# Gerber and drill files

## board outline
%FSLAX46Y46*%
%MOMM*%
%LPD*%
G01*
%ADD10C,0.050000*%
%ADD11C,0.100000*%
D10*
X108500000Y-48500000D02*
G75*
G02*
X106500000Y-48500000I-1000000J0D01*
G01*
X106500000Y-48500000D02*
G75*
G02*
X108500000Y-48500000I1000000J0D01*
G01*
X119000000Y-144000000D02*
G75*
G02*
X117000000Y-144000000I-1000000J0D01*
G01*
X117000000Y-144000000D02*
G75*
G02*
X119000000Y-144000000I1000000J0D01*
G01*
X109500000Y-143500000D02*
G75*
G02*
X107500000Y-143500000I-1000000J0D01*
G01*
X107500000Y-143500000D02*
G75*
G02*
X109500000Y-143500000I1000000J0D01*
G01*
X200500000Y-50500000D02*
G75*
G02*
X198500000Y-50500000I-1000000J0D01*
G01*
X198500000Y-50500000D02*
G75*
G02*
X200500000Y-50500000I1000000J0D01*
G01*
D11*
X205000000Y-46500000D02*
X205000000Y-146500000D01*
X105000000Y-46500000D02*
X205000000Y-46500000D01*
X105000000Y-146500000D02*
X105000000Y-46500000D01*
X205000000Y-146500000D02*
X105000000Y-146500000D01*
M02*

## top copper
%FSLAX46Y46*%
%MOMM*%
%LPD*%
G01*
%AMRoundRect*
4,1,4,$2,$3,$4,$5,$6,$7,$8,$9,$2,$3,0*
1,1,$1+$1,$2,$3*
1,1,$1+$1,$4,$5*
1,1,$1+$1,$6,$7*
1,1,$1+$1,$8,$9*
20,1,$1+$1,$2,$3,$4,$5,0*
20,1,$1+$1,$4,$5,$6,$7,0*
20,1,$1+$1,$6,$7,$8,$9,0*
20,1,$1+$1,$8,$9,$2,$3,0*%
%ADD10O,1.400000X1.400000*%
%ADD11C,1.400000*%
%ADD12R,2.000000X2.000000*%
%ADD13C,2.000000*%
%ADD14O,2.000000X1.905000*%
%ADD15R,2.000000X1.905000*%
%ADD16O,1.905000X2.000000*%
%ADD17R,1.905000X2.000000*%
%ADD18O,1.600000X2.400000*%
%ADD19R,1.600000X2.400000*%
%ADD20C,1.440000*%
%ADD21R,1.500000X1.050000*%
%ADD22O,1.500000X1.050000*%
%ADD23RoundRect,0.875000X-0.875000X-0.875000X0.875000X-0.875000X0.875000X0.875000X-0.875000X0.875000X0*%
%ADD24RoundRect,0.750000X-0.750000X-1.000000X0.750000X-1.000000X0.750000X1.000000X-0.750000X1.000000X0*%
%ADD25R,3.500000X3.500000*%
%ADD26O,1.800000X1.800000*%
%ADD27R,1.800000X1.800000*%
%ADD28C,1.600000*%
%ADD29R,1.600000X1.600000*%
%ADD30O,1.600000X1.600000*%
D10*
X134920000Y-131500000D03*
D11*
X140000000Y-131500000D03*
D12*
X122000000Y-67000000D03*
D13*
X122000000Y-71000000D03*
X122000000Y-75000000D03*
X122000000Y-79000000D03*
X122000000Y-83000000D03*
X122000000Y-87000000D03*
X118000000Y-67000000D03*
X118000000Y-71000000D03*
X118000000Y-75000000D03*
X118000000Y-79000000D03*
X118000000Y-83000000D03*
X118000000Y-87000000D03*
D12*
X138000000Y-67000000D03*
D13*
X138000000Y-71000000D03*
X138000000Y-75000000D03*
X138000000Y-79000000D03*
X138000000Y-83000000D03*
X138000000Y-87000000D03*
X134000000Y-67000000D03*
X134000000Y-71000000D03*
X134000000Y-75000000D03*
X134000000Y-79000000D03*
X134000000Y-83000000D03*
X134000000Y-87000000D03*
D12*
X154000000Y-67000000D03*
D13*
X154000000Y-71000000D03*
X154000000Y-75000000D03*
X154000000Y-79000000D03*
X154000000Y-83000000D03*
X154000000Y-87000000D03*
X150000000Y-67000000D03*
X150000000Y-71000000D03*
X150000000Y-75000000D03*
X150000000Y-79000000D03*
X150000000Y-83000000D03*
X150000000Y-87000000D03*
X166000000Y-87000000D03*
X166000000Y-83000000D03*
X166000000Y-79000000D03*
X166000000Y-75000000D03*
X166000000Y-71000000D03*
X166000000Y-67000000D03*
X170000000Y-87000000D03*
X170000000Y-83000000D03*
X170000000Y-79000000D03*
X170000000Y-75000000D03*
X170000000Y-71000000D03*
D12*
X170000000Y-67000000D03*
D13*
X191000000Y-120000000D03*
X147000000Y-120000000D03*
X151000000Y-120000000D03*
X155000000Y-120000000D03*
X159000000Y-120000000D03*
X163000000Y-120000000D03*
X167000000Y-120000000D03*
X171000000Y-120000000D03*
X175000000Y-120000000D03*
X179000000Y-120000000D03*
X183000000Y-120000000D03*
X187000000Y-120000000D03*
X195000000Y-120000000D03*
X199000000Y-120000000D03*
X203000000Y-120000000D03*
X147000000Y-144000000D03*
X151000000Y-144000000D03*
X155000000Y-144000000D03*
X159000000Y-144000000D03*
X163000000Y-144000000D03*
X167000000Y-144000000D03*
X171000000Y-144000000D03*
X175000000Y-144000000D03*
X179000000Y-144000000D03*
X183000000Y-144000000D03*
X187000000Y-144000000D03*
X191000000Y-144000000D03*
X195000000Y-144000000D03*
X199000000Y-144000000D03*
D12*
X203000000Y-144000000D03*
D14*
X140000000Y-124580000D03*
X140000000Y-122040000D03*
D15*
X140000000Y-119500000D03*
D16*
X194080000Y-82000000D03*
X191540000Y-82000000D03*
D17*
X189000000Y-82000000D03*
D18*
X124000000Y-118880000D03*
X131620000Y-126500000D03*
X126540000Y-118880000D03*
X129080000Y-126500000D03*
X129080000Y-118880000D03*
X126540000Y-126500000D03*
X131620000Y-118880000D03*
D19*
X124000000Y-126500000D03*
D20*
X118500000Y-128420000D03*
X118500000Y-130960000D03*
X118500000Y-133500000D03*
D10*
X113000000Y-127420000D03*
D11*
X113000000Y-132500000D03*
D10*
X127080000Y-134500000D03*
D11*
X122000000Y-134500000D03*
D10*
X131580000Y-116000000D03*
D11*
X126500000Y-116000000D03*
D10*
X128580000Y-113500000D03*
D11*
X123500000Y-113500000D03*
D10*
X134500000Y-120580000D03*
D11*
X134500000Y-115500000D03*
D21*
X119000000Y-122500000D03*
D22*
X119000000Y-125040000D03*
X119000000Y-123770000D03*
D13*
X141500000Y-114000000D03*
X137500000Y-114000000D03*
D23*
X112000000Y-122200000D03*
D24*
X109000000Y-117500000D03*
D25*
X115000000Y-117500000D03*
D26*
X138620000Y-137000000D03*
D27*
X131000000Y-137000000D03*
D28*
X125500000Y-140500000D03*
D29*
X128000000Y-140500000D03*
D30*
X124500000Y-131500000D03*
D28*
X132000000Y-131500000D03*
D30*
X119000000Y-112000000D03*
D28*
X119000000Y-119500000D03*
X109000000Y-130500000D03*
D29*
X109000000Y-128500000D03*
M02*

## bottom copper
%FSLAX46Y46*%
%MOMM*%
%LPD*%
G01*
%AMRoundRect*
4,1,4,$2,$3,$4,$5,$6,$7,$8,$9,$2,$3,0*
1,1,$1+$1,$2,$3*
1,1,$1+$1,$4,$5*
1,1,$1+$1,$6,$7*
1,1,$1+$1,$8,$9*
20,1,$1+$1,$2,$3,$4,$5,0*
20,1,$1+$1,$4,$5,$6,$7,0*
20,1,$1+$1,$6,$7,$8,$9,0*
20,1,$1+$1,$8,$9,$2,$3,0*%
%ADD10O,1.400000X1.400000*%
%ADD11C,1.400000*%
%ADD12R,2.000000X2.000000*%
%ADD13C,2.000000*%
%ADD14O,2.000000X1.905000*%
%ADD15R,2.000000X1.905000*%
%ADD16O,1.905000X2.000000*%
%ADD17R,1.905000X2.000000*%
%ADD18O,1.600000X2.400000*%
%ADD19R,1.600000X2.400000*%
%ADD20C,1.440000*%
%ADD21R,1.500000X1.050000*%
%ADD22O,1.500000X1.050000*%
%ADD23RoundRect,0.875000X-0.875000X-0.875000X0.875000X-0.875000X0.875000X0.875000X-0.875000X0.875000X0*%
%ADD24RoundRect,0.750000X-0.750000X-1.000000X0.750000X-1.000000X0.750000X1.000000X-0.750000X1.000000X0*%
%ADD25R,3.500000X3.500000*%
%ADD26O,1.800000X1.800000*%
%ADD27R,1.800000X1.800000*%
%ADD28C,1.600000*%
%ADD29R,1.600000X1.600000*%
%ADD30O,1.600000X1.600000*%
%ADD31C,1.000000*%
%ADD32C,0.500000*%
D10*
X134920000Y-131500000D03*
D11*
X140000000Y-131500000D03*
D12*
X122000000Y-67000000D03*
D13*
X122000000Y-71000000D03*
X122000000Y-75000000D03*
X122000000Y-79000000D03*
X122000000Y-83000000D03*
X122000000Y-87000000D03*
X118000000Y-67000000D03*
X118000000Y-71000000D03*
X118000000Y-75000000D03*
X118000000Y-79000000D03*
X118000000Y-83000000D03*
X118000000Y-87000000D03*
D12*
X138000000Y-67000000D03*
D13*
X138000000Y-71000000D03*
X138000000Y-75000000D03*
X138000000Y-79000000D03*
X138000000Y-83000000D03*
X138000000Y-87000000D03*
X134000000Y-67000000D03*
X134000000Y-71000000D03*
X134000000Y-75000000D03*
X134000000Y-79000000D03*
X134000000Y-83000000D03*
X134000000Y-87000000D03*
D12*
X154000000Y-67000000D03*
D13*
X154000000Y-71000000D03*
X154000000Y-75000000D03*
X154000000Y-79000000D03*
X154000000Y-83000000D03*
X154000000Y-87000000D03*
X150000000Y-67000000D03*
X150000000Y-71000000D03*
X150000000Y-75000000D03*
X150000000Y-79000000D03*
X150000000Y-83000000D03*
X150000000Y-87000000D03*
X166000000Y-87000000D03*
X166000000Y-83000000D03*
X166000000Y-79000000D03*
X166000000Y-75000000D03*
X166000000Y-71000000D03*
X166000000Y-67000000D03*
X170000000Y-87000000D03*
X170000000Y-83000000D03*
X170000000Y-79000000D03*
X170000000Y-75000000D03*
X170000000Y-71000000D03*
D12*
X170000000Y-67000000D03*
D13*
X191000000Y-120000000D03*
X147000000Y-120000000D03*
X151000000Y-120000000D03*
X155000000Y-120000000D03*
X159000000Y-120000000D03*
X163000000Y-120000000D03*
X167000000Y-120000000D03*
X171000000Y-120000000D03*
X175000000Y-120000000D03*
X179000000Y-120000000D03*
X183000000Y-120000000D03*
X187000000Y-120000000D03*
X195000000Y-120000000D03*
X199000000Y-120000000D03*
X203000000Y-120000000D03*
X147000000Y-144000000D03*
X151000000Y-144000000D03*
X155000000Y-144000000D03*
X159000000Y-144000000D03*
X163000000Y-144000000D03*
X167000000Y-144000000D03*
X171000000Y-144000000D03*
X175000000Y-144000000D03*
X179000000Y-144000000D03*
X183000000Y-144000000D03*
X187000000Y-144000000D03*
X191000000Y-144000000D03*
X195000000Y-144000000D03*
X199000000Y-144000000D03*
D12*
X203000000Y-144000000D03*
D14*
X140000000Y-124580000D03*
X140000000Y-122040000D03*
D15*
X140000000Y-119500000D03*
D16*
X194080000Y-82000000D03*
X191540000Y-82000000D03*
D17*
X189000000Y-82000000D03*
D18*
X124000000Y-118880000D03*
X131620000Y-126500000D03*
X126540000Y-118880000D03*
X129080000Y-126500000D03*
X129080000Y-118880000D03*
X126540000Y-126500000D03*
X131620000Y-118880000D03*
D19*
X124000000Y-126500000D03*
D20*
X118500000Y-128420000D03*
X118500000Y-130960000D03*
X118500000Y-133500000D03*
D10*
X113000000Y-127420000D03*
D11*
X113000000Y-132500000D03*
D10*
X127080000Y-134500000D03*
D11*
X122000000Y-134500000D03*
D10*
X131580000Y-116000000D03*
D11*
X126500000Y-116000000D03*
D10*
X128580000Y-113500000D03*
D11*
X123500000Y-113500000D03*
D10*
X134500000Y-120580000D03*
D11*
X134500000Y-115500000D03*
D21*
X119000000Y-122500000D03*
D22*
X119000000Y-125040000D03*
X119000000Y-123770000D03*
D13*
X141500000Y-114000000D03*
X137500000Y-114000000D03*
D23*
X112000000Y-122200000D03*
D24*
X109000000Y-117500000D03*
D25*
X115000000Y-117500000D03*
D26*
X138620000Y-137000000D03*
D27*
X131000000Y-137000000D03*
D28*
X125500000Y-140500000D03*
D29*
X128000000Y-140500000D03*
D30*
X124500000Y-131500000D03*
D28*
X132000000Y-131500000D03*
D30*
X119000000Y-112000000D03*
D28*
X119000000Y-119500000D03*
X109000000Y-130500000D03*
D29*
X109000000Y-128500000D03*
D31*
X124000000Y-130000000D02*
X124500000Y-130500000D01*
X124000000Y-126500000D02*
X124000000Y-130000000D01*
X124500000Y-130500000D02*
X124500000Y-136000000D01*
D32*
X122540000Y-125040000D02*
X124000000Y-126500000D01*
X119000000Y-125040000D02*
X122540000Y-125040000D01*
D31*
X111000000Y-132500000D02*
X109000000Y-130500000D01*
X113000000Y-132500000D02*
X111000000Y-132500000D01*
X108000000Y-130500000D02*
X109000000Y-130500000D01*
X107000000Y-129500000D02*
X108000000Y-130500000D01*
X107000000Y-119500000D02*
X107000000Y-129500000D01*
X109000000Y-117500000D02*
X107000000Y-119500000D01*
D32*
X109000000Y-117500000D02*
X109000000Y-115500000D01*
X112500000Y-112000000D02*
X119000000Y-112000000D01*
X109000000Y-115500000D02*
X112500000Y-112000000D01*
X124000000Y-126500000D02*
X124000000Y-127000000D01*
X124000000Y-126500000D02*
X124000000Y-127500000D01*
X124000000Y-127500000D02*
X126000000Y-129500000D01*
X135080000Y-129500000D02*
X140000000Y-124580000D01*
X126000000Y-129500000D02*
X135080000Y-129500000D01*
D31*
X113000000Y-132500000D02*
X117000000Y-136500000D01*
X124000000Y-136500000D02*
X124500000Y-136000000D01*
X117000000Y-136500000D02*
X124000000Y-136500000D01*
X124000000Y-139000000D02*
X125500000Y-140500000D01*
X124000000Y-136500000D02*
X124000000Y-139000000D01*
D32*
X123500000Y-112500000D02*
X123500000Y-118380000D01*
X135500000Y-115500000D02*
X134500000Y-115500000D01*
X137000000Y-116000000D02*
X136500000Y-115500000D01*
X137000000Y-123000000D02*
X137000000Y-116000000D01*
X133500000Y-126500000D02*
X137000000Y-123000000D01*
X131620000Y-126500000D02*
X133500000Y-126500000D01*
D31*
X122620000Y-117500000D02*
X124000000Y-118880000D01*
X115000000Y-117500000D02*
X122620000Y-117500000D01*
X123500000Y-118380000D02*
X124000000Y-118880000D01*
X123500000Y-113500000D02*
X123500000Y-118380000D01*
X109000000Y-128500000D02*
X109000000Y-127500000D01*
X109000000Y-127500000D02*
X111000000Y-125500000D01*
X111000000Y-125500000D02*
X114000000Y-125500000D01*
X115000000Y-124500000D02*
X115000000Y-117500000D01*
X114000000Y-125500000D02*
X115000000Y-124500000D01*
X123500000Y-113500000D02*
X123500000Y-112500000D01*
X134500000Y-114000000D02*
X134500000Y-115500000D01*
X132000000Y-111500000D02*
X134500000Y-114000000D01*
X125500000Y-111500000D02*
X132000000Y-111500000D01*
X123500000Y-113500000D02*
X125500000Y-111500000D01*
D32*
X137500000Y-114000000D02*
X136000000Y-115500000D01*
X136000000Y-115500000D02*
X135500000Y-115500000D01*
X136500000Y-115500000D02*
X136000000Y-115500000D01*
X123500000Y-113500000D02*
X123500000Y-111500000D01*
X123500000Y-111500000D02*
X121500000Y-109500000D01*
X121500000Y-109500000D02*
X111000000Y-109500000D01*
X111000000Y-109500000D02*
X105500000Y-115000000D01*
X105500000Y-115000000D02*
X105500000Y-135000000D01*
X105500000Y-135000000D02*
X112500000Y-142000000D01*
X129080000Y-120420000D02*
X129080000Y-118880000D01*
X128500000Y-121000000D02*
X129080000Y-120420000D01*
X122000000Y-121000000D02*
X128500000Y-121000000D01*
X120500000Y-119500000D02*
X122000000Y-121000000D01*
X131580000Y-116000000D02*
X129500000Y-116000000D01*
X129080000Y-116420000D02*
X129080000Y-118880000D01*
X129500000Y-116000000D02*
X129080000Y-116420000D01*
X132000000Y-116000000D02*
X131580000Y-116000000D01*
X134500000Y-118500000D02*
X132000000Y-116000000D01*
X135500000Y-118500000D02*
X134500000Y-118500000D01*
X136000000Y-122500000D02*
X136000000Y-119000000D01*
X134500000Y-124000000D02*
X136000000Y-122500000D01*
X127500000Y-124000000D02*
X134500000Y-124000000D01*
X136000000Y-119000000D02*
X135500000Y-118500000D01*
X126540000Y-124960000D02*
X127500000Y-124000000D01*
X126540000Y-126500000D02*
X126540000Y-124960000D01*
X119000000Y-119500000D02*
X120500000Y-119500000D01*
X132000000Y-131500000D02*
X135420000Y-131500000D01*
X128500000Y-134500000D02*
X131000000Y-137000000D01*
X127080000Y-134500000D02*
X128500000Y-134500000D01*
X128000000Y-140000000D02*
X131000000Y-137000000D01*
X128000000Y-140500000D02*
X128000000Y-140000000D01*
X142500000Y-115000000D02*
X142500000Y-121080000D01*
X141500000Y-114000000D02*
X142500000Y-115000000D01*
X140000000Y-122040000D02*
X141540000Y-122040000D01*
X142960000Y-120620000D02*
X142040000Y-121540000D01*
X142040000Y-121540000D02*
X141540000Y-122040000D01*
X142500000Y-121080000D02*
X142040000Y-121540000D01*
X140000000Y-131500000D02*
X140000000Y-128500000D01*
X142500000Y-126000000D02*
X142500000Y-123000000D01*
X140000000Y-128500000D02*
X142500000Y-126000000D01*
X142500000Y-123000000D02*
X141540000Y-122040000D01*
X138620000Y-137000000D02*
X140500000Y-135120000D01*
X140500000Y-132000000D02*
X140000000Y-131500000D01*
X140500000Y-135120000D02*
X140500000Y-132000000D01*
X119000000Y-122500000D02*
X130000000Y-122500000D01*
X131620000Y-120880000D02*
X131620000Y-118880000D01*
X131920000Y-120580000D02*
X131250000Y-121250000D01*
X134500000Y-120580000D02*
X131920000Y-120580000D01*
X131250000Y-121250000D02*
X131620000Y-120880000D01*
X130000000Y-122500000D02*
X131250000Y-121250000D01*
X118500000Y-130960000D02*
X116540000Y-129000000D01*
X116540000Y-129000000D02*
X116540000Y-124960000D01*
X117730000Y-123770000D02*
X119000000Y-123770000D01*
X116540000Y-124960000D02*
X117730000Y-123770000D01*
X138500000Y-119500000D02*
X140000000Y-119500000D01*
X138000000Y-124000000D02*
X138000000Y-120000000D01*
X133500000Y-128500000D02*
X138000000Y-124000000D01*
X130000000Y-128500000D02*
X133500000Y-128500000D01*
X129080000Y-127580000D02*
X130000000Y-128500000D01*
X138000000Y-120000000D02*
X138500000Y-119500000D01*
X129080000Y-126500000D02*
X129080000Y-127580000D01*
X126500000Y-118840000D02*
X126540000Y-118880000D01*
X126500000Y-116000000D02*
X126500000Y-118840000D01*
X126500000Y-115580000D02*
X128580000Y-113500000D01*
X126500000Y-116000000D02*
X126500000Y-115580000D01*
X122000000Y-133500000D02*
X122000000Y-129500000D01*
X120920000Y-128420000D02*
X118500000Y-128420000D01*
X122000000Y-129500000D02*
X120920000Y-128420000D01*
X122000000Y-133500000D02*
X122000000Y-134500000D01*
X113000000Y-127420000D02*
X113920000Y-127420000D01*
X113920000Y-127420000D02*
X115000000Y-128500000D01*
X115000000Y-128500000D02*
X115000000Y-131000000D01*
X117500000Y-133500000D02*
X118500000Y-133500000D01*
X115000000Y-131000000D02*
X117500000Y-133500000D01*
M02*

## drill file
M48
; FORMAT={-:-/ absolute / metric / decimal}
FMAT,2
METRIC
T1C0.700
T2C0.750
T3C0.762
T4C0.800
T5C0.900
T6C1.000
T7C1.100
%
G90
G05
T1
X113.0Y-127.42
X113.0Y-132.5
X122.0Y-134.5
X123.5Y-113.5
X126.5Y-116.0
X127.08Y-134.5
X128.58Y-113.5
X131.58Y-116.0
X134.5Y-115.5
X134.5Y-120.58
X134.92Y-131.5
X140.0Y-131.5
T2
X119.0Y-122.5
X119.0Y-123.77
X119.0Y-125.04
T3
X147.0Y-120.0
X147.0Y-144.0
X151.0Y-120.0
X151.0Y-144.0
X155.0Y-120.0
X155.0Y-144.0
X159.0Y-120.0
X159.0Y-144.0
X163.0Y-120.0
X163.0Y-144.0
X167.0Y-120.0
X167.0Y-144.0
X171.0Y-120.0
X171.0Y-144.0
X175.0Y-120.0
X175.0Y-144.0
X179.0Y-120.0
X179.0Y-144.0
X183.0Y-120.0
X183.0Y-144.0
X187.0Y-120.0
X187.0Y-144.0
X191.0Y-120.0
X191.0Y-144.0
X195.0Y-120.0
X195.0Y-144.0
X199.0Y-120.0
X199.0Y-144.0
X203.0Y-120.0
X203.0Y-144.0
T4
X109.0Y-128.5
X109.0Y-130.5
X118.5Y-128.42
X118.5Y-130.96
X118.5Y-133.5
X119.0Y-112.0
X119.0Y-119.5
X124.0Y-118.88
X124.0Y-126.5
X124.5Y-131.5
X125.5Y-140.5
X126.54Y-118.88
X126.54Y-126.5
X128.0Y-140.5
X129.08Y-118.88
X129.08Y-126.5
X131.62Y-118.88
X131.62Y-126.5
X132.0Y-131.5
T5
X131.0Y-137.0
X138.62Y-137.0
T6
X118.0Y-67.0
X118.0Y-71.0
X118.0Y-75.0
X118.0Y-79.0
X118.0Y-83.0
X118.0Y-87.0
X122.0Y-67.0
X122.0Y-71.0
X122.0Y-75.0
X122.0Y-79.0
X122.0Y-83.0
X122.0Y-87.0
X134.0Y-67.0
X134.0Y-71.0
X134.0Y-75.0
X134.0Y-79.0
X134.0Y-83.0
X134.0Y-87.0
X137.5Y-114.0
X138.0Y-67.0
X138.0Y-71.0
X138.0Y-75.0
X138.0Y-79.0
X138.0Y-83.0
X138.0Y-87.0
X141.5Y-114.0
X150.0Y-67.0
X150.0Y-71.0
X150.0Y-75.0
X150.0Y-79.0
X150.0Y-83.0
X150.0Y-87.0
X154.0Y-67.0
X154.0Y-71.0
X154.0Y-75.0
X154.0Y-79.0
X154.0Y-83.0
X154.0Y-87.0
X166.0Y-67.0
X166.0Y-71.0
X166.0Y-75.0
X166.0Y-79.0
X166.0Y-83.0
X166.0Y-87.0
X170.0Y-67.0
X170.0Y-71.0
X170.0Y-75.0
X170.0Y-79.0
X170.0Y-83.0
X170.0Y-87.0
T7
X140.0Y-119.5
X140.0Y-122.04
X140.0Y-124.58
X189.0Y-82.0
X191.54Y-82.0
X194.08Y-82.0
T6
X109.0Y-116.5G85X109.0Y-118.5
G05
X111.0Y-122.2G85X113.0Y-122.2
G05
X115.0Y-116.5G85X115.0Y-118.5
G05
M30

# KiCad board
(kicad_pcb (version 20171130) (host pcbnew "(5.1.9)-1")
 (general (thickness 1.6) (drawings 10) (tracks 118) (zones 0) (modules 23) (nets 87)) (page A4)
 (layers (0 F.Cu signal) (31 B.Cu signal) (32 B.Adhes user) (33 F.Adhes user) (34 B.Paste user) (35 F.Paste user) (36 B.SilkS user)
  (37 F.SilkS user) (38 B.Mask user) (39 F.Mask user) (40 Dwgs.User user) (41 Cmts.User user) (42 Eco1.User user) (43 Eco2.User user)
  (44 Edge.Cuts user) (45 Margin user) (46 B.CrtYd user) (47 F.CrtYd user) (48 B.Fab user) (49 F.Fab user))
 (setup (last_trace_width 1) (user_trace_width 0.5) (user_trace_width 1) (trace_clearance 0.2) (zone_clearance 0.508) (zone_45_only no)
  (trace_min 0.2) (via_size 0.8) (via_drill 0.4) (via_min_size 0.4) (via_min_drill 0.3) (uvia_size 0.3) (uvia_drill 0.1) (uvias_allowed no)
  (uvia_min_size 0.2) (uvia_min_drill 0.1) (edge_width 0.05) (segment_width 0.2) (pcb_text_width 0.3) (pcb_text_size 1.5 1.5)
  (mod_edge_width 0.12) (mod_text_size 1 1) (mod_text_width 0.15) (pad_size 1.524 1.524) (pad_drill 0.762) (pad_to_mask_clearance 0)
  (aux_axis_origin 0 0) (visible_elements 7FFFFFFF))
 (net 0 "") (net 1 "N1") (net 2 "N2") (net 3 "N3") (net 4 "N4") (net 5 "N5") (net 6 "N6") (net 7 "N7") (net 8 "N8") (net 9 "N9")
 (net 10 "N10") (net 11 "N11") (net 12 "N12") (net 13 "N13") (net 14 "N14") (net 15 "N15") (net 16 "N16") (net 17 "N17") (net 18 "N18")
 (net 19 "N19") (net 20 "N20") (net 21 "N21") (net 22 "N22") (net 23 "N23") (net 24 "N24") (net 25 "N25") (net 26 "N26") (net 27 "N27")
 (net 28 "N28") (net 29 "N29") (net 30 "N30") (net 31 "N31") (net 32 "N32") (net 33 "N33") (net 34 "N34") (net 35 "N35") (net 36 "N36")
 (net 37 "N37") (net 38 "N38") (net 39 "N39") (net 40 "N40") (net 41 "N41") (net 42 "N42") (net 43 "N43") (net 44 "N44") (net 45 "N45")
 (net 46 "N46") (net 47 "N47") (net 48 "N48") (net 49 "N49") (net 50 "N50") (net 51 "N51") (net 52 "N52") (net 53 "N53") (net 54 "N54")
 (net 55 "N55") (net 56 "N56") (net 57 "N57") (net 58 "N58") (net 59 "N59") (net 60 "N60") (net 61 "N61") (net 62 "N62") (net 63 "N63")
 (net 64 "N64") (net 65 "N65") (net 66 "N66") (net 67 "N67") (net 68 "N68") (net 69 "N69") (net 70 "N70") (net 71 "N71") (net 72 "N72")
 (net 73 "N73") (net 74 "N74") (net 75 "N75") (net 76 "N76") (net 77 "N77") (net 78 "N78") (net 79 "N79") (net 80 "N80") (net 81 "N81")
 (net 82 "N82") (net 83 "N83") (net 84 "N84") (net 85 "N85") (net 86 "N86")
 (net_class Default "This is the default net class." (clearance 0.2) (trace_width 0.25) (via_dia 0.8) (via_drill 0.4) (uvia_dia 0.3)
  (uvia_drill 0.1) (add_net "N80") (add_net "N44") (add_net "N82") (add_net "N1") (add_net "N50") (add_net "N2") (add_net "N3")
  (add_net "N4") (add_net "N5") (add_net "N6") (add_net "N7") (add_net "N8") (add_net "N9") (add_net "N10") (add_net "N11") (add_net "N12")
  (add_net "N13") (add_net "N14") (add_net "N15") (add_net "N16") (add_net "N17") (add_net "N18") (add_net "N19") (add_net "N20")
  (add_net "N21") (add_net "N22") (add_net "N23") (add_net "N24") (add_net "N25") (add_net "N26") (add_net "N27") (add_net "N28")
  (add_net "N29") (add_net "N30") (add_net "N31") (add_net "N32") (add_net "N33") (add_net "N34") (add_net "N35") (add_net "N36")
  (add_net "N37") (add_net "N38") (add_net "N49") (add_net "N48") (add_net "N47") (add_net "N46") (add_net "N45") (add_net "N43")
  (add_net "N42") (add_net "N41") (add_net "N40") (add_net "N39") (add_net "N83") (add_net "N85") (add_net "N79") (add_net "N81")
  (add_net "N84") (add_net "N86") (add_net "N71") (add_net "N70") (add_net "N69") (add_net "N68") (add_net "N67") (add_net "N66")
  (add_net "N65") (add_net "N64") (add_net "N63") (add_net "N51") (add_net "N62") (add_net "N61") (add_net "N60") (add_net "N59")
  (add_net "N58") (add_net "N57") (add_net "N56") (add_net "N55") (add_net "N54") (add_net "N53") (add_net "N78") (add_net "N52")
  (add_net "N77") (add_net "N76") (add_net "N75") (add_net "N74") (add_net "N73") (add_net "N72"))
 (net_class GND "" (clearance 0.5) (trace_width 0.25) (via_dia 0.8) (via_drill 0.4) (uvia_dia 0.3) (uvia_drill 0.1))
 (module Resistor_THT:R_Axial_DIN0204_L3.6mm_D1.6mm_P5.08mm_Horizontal (layer F.Cu) (at 140 131.5 180)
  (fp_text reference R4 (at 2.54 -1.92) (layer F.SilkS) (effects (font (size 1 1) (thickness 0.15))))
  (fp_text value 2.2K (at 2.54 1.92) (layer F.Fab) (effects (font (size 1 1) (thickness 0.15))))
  (pad 2 thru_hole oval (at 5.08 0 180) (size 1.4 1.4) (drill 0.7) (layers *.Cu *.Mask) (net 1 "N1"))
  (pad 1 thru_hole circle (at 0 0 180) (size 1.4 1.4) (drill 0.7) (layers *.Cu *.Mask) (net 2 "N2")))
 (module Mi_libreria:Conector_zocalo (layer F.Cu) (at 120 67 180)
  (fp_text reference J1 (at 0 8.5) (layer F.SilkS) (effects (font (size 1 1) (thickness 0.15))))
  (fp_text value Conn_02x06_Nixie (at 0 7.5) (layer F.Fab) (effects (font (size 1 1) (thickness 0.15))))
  (pad 1 thru_hole rect (at -2 0 180) (size 2 2) (drill 1) (layers *.Cu *.Mask) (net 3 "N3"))
  (pad 2 thru_hole circle (at -2 -4 180) (size 2 2) (drill 1) (layers *.Cu *.Mask) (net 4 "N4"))
  (pad 3 thru_hole circle (at -2 -8 180) (size 2 2) (drill 1) (layers *.Cu *.Mask) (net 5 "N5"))
  (pad 4 thru_hole circle (at -2 -12 180) (size 2 2) (drill 1) (layers *.Cu *.Mask) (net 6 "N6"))
  (pad 5 thru_hole circle (at -2 -16 180) (size 2 2) (drill 1) (layers *.Cu *.Mask) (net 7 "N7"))
  (pad 6 thru_hole circle (at -2 -20 180) (size 2 2) (drill 1) (layers *.Cu *.Mask) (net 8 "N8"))
  (pad A thru_hole circle (at 2 0 180) (size 2 2) (drill 1) (layers *.Cu *.Mask) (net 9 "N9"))
  (pad B thru_hole circle (at 2 -4 180) (size 2 2) (drill 1) (layers *.Cu *.Mask) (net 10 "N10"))
  (pad C thru_hole circle (at 2 -8 180) (size 2 2) (drill 1) (layers *.Cu *.Mask) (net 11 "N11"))
  (pad D thru_hole circle (at 2 -12 180) (size 2 2) (drill 1) (layers *.Cu *.Mask) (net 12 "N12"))
  (pad E thru_hole circle (at 2 -16 180) (size 2 2) (drill 1) (layers *.Cu *.Mask) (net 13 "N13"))
  (pad F thru_hole circle (at 2 -20 180) (size 2 2) (drill 1) (layers *.Cu *.Mask) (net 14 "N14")))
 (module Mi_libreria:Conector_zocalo (layer F.Cu) (at 136 67 180)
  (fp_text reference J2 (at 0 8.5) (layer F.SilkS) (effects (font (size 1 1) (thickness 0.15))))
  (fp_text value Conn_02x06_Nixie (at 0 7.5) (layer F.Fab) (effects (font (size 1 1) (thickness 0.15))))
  (pad 1 thru_hole rect (at -2 0 180) (size 2 2) (drill 1) (layers *.Cu *.Mask) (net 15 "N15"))
  (pad 2 thru_hole circle (at -2 -4 180) (size 2 2) (drill 1) (layers *.Cu *.Mask) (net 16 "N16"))
  (pad 3 thru_hole circle (at -2 -8 180) (size 2 2) (drill 1) (layers *.Cu *.Mask) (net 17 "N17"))
  (pad 4 thru_hole circle (at -2 -12 180) (size 2 2) (drill 1) (layers *.Cu *.Mask) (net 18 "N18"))
  (pad 5 thru_hole circle (at -2 -16 180) (size 2 2) (drill 1) (layers *.Cu *.Mask) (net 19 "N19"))
  (pad 6 thru_hole circle (at -2 -20 180) (size 2 2) (drill 1) (layers *.Cu *.Mask) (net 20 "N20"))
  (pad A thru_hole circle (at 2 0 180) (size 2 2) (drill 1) (layers *.Cu *.Mask) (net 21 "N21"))
  (pad B thru_hole circle (at 2 -4 180) (size 2 2) (drill 1) (layers *.Cu *.Mask) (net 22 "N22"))
  (pad C thru_hole circle (at 2 -8 180) (size 2 2) (drill 1) (layers *.Cu *.Mask) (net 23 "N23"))
  (pad D thru_hole circle (at 2 -12 180) (size 2 2) (drill 1) (layers *.Cu *.Mask) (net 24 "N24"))
  (pad E thru_hole circle (at 2 -16 180) (size 2 2) (drill 1) (layers *.Cu *.Mask) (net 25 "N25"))
  (pad F thru_hole circle (at 2 -20 180) (size 2 2) (drill 1) (layers *.Cu *.Mask) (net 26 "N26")))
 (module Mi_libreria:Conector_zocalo (layer F.Cu) (at 152 67 180)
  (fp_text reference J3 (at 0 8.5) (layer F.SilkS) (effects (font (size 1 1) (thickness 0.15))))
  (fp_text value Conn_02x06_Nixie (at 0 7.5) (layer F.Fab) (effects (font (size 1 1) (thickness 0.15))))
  (pad 1 thru_hole rect (at -2 0 180) (size 2 2) (drill 1) (layers *.Cu *.Mask) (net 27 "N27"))
  (pad 2 thru_hole circle (at -2 -4 180) (size 2 2) (drill 1) (layers *.Cu *.Mask) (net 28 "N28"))
  (pad 3 thru_hole circle (at -2 -8 180) (size 2 2) (drill 1) (layers *.Cu *.Mask) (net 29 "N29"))
  (pad 4 thru_hole circle (at -2 -12 180) (size 2 2) (drill 1) (layers *.Cu *.Mask) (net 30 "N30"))
  (pad 5 thru_hole circle (at -2 -16 180) (size 2 2) (drill 1) (layers *.Cu *.Mask) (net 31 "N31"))
  (pad 6 thru_hole circle (at -2 -20 180) (size 2 2) (drill 1) (layers *.Cu *.Mask) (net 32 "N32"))
  (pad A thru_hole circle (at 2 0 180) (size 2 2) (drill 1) (layers *.Cu *.Mask) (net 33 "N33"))
  (pad B thru_hole circle (at 2 -4 180) (size 2 2) (drill 1) (layers *.Cu *.Mask) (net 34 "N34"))
  (pad C thru_hole circle (at 2 -8 180) (size 2 2) (drill 1) (layers *.Cu *.Mask) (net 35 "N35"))
  (pad D thru_hole circle (at 2 -12 180) (size 2 2) (drill 1) (layers *.Cu *.Mask) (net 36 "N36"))
  (pad E thru_hole circle (at 2 -16 180) (size 2 2) (drill 1) (layers *.Cu *.Mask) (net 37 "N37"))
  (pad F thru_hole circle (at 2 -20 180) (size 2 2) (drill 1) (layers *.Cu *.Mask) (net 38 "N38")))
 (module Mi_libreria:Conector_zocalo (layer F.Cu) (at 168 67 180)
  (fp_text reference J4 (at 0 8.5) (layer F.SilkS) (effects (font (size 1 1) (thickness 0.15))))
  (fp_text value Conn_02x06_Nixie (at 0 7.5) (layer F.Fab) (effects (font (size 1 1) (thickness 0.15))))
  (pad F thru_hole circle (at 2 -20 180) (size 2 2) (drill 1) (layers *.Cu *.Mask) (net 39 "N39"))
  (pad E thru_hole circle (at 2 -16 180) (size 2 2) (drill 1) (layers *.Cu *.Mask) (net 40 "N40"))
  (pad D thru_hole circle (at 2 -12 180) (size 2 2) (drill 1) (layers *.Cu *.Mask) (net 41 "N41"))
  (pad C thru_hole circle (at 2 -8 180) (size 2 2) (drill 1) (layers *.Cu *.Mask) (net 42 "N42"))
  (pad B thru_hole circle (at 2 -4 180) (size 2 2) (drill 1) (layers *.Cu *.Mask) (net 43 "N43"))
  (pad A thru_hole circle (at 2 0 180) (size 2 2) (drill 1) (layers *.Cu *.Mask) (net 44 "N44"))
  (pad 6 thru_hole circle (at -2 -20 180) (size 2 2) (drill 1) (layers *.Cu *.Mask) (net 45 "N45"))
  (pad 5 thru_hole circle (at -2 -16 180) (size 2 2) (drill 1) (layers *.Cu *.Mask) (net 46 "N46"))
  (pad 4 thru_hole circle (at -2 -12 180) (size 2 2) (drill 1) (layers *.Cu *.Mask) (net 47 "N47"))
  (pad 3 thru_hole circle (at -2 -8 180) (size 2 2) (drill 1) (layers *.Cu *.Mask) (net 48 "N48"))
  (pad 2 thru_hole circle (at -2 -4 180) (size 2 2) (drill 1) (layers *.Cu *.Mask) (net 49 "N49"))
  (pad 1 thru_hole rect (at -2 0 180) (size 2 2) (drill 1) (layers *.Cu *.Mask) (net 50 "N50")))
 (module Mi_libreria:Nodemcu (layer F.Cu) (at 203 132 90)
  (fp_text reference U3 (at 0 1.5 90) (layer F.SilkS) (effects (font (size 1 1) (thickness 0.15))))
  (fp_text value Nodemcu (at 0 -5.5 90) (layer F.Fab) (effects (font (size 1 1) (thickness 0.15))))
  (pad 19 thru_hole circle (at 12 -12 90) (size 2 2) (drill 0.762) (layers *.Cu *.Mask) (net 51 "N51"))
  (pad 30 thru_hole circle (at 12 -56 90) (size 2 2) (drill 0.762) (layers *.Cu *.Mask) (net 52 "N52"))
  (pad 29 thru_hole circle (at 12 -52 90) (size 2 2) (drill 0.762) (layers *.Cu *.Mask) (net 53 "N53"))
  (pad 28 thru_hole circle (at 12 -48 90) (size 2 2) (drill 0.762) (layers *.Cu *.Mask) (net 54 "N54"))
  (pad 27 thru_hole circle (at 12 -44 90) (size 2 2) (drill 0.762) (layers *.Cu *.Mask) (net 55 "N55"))
  (pad 26 thru_hole circle (at 12 -40 90) (size 2 2) (drill 0.762) (layers *.Cu *.Mask) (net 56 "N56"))
  (pad 25 thru_hole circle (at 12 -36 90) (size 2 2) (drill 0.762) (layers *.Cu *.Mask) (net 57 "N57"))
  (pad 24 thru_hole circle (at 12 -32 90) (size 2 2) (drill 0.762) (layers *.Cu *.Mask) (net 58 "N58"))
  (pad 23 thru_hole circle (at 12 -28 90) (size 2 2) (drill 0.762) (layers *.Cu *.Mask) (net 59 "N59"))
  (pad 22 thru_hole circle (at 12 -24 90) (size 2 2) (drill 0.762) (layers *.Cu *.Mask) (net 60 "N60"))
  (pad 21 thru_hole circle (at 12 -20 90) (size 2 2) (drill 0.762) (layers *.Cu *.Mask) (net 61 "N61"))
  (pad 20 thru_hole circle (at 12 -16 90) (size 2 2) (drill 0.762) (layers *.Cu *.Mask) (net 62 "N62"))
  (pad 18 thru_hole circle (at 12 -8 90) (size 2 2) (drill 0.762) (layers *.Cu *.Mask) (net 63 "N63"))
  (pad 17 thru_hole circle (at 12 -4 90) (size 2 2) (drill 0.762) (layers *.Cu *.Mask) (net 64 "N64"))
  (pad 16 thru_hole circle (at 12 0 90) (size 2 2) (drill 0.762) (layers *.Cu *.Mask) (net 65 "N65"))
  (pad 15 thru_hole circle (at -12 -56 90) (size 2 2) (drill 0.762) (layers *.Cu *.Mask) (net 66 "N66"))
  (pad 14 thru_hole circle (at -12 -52 90) (size 2 2) (drill 0.762) (layers *.Cu *.Mask) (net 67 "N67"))
  (pad 13 thru_hole circle (at -12 -48 90) (size 2 2) (drill 0.762) (layers *.Cu *.Mask) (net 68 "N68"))
  (pad 12 thru_hole circle (at -12 -44 90) (size 2 2) (drill 0.762) (layers *.Cu *.Mask) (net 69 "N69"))
  (pad 11 thru_hole circle (at -12 -40 90) (size 2 2) (drill 0.762) (layers *.Cu *.Mask) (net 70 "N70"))
  (pad 10 thru_hole circle (at -12 -36 90) (size 2 2) (drill 0.762) (layers *.Cu *.Mask) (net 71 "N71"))
  (pad 9 thru_hole circle (at -12 -32 90) (size 2 2) (drill 0.762) (layers *.Cu *.Mask) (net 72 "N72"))
  (pad 8 thru_hole circle (at -12 -28 90) (size 2 2) (drill 0.762) (layers *.Cu *.Mask) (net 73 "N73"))
  (pad 7 thru_hole circle (at -12 -24 90) (size 2 2) (drill 0.762) (layers *.Cu *.Mask) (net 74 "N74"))
  (pad 6 thru_hole circle (at -12 -20 90) (size 2 2) (drill 0.762) (layers *.Cu *.Mask) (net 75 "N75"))
  (pad 5 thru_hole circle (at -12 -16 90) (size 2 2) (drill 0.762) (layers *.Cu *.Mask) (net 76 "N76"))
  (pad 4 thru_hole circle (at -12 -12 90) (size 2 2) (drill 0.762) (layers *.Cu *.Mask) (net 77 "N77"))
  (pad 3 thru_hole circle (at -12 -8 90) (size 2 2) (drill 0.762) (layers *.Cu *.Mask) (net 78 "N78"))
  (pad 2 thru_hole circle (at -12 -4 90) (size 2 2) (drill 0.762) (layers *.Cu *.Mask) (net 44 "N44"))
  (pad 1 thru_hole rect (at -12 0 90) (size 2 2) (drill 0.762) (layers *.Cu *.Mask) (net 49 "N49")))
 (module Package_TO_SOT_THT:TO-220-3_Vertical (layer F.Cu) (at 140 119.5 270)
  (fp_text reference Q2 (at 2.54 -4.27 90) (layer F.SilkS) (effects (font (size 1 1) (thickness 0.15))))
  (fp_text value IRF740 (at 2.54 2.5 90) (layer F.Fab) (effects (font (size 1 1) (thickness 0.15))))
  (pad 3 thru_hole oval (at 5.08 0 270) (size 1.905 2) (drill 1.1) (layers *.Cu *.Mask) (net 44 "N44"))
  (pad 2 thru_hole oval (at 2.54 0 270) (size 1.905 2) (drill 1.1) (layers *.Cu *.Mask) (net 2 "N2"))
  (pad 1 thru_hole rect (at 0 0 270) (size 1.905 2) (drill 1.1) (layers *.Cu *.Mask) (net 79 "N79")))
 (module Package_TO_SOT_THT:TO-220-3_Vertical (layer F.Cu) (at 189 82)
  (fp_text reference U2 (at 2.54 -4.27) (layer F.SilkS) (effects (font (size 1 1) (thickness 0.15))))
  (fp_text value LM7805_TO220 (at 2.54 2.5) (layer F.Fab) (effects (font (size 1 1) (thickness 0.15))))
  (pad 3 thru_hole oval (at 5.08 0) (size 1.905 2) (drill 1.1) (layers *.Cu *.Mask) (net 49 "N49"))
  (pad 2 thru_hole oval (at 2.54 0) (size 1.905 2) (drill 1.1) (layers *.Cu *.Mask) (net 44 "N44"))
  (pad 1 thru_hole rect (at 0 0) (size 1.905 2) (drill 1.1) (layers *.Cu *.Mask) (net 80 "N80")))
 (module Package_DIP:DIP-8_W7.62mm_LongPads (layer F.Cu) (at 124 126.5 90)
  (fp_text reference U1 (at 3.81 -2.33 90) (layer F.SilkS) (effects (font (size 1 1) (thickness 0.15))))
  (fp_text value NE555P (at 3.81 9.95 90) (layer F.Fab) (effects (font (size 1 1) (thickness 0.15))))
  (pad 8 thru_hole oval (at 7.62 0 90) (size 2.4 1.6) (drill 0.8) (layers *.Cu *.Mask) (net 80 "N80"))
  (pad 4 thru_hole oval (at 0 7.62 90) (size 2.4 1.6) (drill 0.8) (layers *.Cu *.Mask) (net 80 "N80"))
  (pad 7 thru_hole oval (at 7.62 2.54 90) (size 2.4 1.6) (drill 0.8) (layers *.Cu *.Mask) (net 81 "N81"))
  (pad 3 thru_hole oval (at 0 5.08 90) (size 2.4 1.6) (drill 0.8) (layers *.Cu *.Mask) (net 79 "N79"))
  (pad 6 thru_hole oval (at 7.62 5.08 90) (size 2.4 1.6) (drill 0.8) (layers *.Cu *.Mask) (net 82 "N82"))
  (pad 2 thru_hole oval (at 0 2.54 90) (size 2.4 1.6) (drill 0.8) (layers *.Cu *.Mask) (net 82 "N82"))
  (pad 5 thru_hole oval (at 7.62 7.62 90) (size 2.4 1.6) (drill 0.8) (layers *.Cu *.Mask) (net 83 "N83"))
  (pad 1 thru_hole rect (at 0 0 90) (size 2.4 1.6) (drill 0.8) (layers *.Cu *.Mask) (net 44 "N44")))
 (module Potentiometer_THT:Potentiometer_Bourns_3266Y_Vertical (layer F.Cu) (at 118.5 133.5 270)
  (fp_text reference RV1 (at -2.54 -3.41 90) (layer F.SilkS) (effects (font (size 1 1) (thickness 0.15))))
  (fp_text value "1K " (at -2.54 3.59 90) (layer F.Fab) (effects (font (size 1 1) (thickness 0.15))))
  (pad 3 thru_hole circle (at -5.08 0 270) (size 1.44 1.44) (drill 0.8) (layers *.Cu *.Mask) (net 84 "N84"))
  (pad 2 thru_hole circle (at -2.54 0 270) (size 1.44 1.44) (drill 0.8) (layers *.Cu *.Mask) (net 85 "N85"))
  (pad 1 thru_hole circle (at 0 0 270) (size 1.44 1.44) (drill 0.8) (layers *.Cu *.Mask) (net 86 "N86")))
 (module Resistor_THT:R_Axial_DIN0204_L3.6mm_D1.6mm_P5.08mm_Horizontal (layer F.Cu) (at 113 132.5 90)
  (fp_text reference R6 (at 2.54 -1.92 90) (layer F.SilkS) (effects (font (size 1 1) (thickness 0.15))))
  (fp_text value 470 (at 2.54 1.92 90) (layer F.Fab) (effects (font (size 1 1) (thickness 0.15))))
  (pad 2 thru_hole oval (at 5.08 0 90) (size 1.4 1.4) (drill 0.7) (layers *.Cu *.Mask) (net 86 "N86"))
  (pad 1 thru_hole circle (at 0 0 90) (size 1.4 1.4) (drill 0.7) (layers *.Cu *.Mask) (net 44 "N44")))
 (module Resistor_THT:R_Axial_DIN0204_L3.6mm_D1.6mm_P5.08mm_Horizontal (layer F.Cu) (at 122 134.5)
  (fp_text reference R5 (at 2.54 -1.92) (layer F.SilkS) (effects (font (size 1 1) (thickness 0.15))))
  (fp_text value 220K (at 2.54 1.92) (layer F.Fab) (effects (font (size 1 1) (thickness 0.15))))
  (pad 2 thru_hole oval (at 5.08 0) (size 1.4 1.4) (drill 0.7) (layers *.Cu *.Mask) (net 50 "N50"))
  (pad 1 thru_hole circle (at 0 0) (size 1.4 1.4) (drill 0.7) (layers *.Cu *.Mask) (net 84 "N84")))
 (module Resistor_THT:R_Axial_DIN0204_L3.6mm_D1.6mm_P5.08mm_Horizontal (layer F.Cu) (at 126.5 116)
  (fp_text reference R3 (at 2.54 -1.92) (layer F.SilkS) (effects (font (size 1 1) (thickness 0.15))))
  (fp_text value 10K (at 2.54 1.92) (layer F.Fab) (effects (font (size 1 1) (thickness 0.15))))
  (pad 2 thru_hole oval (at 5.08 0) (size 1.4 1.4) (drill 0.7) (layers *.Cu *.Mask) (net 82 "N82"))
  (pad 1 thru_hole circle (at 0 0) (size 1.4 1.4) (drill 0.7) (layers *.Cu *.Mask) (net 81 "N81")))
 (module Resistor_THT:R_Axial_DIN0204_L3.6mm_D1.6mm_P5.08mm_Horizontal (layer F.Cu) (at 123.5 113.5)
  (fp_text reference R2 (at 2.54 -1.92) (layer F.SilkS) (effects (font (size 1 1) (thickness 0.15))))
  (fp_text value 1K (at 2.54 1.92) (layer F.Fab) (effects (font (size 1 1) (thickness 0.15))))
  (pad 2 thru_hole oval (at 5.08 0) (size 1.4 1.4) (drill 0.7) (layers *.Cu *.Mask) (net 81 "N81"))
  (pad 1 thru_hole circle (at 0 0) (size 1.4 1.4) (drill 0.7) (layers *.Cu *.Mask) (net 80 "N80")))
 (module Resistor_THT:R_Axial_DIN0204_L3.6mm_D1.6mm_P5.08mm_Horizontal (layer F.Cu) (at 134.5 115.5 270)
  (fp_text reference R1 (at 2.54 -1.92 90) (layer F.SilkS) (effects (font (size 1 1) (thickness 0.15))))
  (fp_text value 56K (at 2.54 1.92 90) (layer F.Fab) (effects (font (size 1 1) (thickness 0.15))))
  (pad 2 thru_hole oval (at 5.08 0 270) (size 1.4 1.4) (drill 0.7) (layers *.Cu *.Mask) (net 83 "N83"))
  (pad 1 thru_hole circle (at 0 0 270) (size 1.4 1.4) (drill 0.7) (layers *.Cu *.Mask) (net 80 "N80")))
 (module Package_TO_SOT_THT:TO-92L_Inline (layer F.Cu) (at 119 122.5 270)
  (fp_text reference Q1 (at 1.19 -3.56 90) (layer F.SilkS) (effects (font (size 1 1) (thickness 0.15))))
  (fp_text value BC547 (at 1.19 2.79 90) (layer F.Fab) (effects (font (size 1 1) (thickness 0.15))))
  (pad 1 thru_hole rect (at 0 0 270) (size 1.05 1.5) (drill 0.75) (layers *.Cu *.Mask) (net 83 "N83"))
  (pad 3 thru_hole oval (at 2.54 0 270) (size 1.05 1.5) (drill 0.75) (layers *.Cu *.Mask) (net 44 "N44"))
  (pad 2 thru_hole oval (at 1.27 0 270) (size 1.05 1.5) (drill 0.75) (layers *.Cu *.Mask) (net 85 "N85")))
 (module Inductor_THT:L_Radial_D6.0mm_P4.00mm (layer F.Cu) (at 137.5 114)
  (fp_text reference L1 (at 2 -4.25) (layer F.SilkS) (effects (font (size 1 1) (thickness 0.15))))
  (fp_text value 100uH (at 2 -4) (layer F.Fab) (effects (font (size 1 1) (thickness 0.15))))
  (pad 2 thru_hole circle (at 4 0) (size 2 2) (drill 1) (layers *.Cu *.Mask) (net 2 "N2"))
  (pad 1 thru_hole circle (at 0 0) (size 2 2) (drill 1) (layers *.Cu *.Mask) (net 80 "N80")))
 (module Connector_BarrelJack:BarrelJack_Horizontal (layer F.Cu) (at 115 117.5)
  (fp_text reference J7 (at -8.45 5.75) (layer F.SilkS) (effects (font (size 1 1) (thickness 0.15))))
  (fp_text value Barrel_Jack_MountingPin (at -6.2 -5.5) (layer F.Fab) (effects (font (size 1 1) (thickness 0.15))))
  (pad 3 thru_hole roundrect (at -3 4.7) (size 3.5 3.5) (drill oval 3 1) (layers *.Cu *.Mask) (roundrect_rratio 0.25))
  (pad 2 thru_hole roundrect (at -6 0) (size 3 3.5) (drill oval 1 3) (layers *.Cu *.Mask) (roundrect_rratio 0.25) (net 44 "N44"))
  (pad 1 thru_hole rect (at 0 0) (size 3.5 3.5) (drill oval 1 3) (layers *.Cu *.Mask) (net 80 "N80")))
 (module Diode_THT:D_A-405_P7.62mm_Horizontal (layer F.Cu) (at 131 137)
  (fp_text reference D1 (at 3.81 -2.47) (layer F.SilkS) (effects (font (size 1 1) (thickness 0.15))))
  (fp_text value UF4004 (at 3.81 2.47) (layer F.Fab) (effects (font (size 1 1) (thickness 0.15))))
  (pad 2 thru_hole oval (at 7.62 0) (size 1.8 1.8) (drill 0.9) (layers *.Cu *.Mask) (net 2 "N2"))
  (pad 1 thru_hole rect (at 0 0) (size 1.8 1.8) (drill 0.9) (layers *.Cu *.Mask) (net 50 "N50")))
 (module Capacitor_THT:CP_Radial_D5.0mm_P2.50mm (layer F.Cu) (at 128 140.5 180)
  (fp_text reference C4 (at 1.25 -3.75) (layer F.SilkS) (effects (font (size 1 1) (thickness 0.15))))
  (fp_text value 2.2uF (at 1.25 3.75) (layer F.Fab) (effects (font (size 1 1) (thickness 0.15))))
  (pad 2 thru_hole circle (at 2.5 0 180) (size 1.6 1.6) (drill 0.8) (layers *.Cu *.Mask) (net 44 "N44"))
  (pad 1 thru_hole rect (at 0 0 180) (size 1.6 1.6) (drill 0.8) (layers *.Cu *.Mask) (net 50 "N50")))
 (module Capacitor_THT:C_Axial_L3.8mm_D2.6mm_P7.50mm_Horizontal (layer F.Cu) (at 132 131.5 180)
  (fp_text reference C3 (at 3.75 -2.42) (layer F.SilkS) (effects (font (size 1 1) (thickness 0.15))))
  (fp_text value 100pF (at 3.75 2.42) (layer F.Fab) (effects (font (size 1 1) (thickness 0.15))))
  (pad 2 thru_hole oval (at 7.5 0 180) (size 1.6 1.6) (drill 0.8) (layers *.Cu *.Mask) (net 44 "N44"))
  (pad 1 thru_hole circle (at 0 0 180) (size 1.6 1.6) (drill 0.8) (layers *.Cu *.Mask) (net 1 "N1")))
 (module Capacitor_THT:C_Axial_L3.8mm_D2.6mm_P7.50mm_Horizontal (layer F.Cu) (at 119 119.5 90)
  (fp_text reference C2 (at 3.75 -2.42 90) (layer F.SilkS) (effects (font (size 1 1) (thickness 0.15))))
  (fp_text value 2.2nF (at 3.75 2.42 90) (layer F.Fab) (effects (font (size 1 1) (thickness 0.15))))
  (pad 2 thru_hole oval (at 7.5 0 90) (size 1.6 1.6) (drill 0.8) (layers *.Cu *.Mask) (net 44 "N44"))
  (pad 1 thru_hole circle (at 0 0 90) (size 1.6 1.6) (drill 0.8) (layers *.Cu *.Mask) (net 82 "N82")))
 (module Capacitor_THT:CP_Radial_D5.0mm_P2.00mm (layer F.Cu) (at 109 128.5 270)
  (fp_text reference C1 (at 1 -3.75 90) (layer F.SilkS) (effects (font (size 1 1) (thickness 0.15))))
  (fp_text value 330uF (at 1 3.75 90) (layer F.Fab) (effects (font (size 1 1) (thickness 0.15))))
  (pad 2 thru_hole circle (at 2 0 270) (size 1.6 1.6) (drill 0.8) (layers *.Cu *.Mask) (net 44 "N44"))
  (pad 1 thru_hole rect (at 0 0 270) (size 1.6 1.6) (drill 0.8) (layers *.Cu *.Mask) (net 80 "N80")))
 (gr_circle (center 107.5 48.5) (end 108.5 48.5) (layer Edge.Cuts) (width 0.05))
 (gr_circle (center 118 144) (end 119 144) (layer Edge.Cuts) (width 0.05))
 (gr_circle (center 108.5 143.5) (end 109.5 143.5) (layer Edge.Cuts) (width 0.05))
 (gr_circle (center 199.5 50.5) (end 200.5 50.5) (layer Edge.Cuts) (width 0.05))
 (gr_line (start 205 46.5) (end 205 146.5) (layer Edge.Cuts) (width 0.1))
 (gr_line (start 105 46.5) (end 205 46.5) (layer Edge.Cuts) (width 0.1))
 (gr_line (start 105 146.5) (end 105 46.5) (layer Edge.Cuts) (width 0.1))
 (gr_line (start 205 146.5) (end 105 146.5) (layer Edge.Cuts) (width 0.1))
 (segment (start 124 130) (end 124.5 130.5) (width 1) (layer B.Cu) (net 44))
 (segment (start 124 126.5) (end 124 130) (width 1) (layer B.Cu) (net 44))
 (segment (start 124.5 130.5) (end 124.5 136) (width 1) (layer B.Cu) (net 44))
 (segment (start 122.54 125.04) (end 124 126.5) (width 0.5) (layer B.Cu) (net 44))
 (segment (start 119 125.04) (end 122.54 125.04) (width 0.5) (layer B.Cu) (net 44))
 (segment (start 111 132.5) (end 109 130.5) (width 1) (layer B.Cu) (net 44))
 (segment (start 113 132.5) (end 111 132.5) (width 1) (layer B.Cu) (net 44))
 (segment (start 108 130.5) (end 109 130.5) (width 1) (layer B.Cu) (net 44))
 (segment (start 107 129.5) (end 108 130.5) (width 1) (layer B.Cu) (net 44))
 (segment (start 107 119.5) (end 107 129.5) (width 1) (layer B.Cu) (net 44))
 (segment (start 109 117.5) (end 107 119.5) (width 1) (layer B.Cu) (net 44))
 (segment (start 109 117.5) (end 109 115.5) (width 0.5) (layer B.Cu) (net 44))
 (segment (start 112.5 112) (end 119 112) (width 0.5) (layer B.Cu) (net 44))
 (segment (start 109 115.5) (end 112.5 112) (width 0.5) (layer B.Cu) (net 44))
 (segment (start 124 126.5) (end 124 127) (width 0.5) (layer B.Cu) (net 44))
 (segment (start 124 126.5) (end 124 127.5) (width 0.5) (layer B.Cu) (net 44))
 (segment (start 124 127.5) (end 126 129.5) (width 0.5) (layer B.Cu) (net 44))
 (segment (start 135.08 129.5) (end 140 124.58) (width 0.5) (layer B.Cu) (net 44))
 (segment (start 126 129.5) (end 135.08 129.5) (width 0.5) (layer B.Cu) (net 44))
 (segment (start 113 132.5) (end 117 136.5) (width 1) (layer B.Cu) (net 44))
 (segment (start 124 136.5) (end 124.5 136) (width 1) (layer B.Cu) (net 44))
 (segment (start 117 136.5) (end 124 136.5) (width 1) (layer B.Cu) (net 44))
 (segment (start 124 139) (end 125.5 140.5) (width 1) (layer B.Cu) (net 44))
 (segment (start 124 136.5) (end 124 139) (width 1) (layer B.Cu) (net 44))
 (segment (start 123.5 112.5) (end 123.5 118.38) (width 0.5) (layer B.Cu) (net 80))
 (segment (start 135.5 115.5) (end 134.5 115.5) (width 0.5) (layer B.Cu) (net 80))
 (segment (start 137 116) (end 136.5 115.5) (width 0.5) (layer B.Cu) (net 80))
 (segment (start 137 123) (end 137 116) (width 0.5) (layer B.Cu) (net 80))
 (segment (start 133.5 126.5) (end 137 123) (width 0.5) (layer B.Cu) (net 80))
 (segment (start 131.62 126.5) (end 133.5 126.5) (width 0.5) (layer B.Cu) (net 80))
 (segment (start 122.62 117.5) (end 124 118.88) (width 1) (layer B.Cu) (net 80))
 (segment (start 115 117.5) (end 122.62 117.5) (width 1) (layer B.Cu) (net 80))
 (segment (start 123.5 118.38) (end 124 118.88) (width 1) (layer B.Cu) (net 80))
 (segment (start 123.5 113.5) (end 123.5 118.38) (width 1) (layer B.Cu) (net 80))
 (segment (start 109 128.5) (end 109 127.5) (width 1) (layer B.Cu) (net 80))
 (segment (start 109 127.5) (end 111 125.5) (width 1) (layer B.Cu) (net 80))
 (segment (start 111 125.5) (end 114 125.5) (width 1) (layer B.Cu) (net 80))
 (segment (start 115 124.5) (end 115 117.5) (width 1) (layer B.Cu) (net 80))
 (segment (start 114 125.5) (end 115 124.5) (width 1) (layer B.Cu) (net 80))
 (segment (start 123.5 113.5) (end 123.5 112.5) (width 1) (layer B.Cu) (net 80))
 (segment (start 134.5 114) (end 134.5 115.5) (width 1) (layer B.Cu) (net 80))
 (segment (start 132 111.5) (end 134.5 114) (width 1) (layer B.Cu) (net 80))
 (segment (start 125.5 111.5) (end 132 111.5) (width 1) (layer B.Cu) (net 80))
 (segment (start 123.5 113.5) (end 125.5 111.5) (width 1) (layer B.Cu) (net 80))
 (segment (start 137.5 114) (end 136 115.5) (width 0.5) (layer B.Cu) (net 80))
 (segment (start 136 115.5) (end 135.5 115.5) (width 0.5) (layer B.Cu) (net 80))
 (segment (start 136.5 115.5) (end 136 115.5) (width 0.5) (layer B.Cu) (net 80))
 (segment (start 123.5 113.5) (end 123.5 111.5) (width 0.5) (layer B.Cu) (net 80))
 (segment (start 123.5 111.5) (end 121.5 109.5) (width 0.5) (layer B.Cu) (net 80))
 (segment (start 121.5 109.5) (end 111 109.5) (width 0.5) (layer B.Cu) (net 80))
 (segment (start 111 109.5) (end 105.5 115) (width 0.5) (layer B.Cu) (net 80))
 (segment (start 105.5 115) (end 105.5 135) (width 0.5) (layer B.Cu) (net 80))
 (segment (start 105.5 135) (end 112.5 142) (width 0.5) (layer B.Cu) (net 80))
 (segment (start 129.08 120.42) (end 129.08 118.88) (width 0.5) (layer B.Cu) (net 82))
 (segment (start 128.5 121) (end 129.08 120.42) (width 0.5) (layer B.Cu) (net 82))
 (segment (start 122 121) (end 128.5 121) (width 0.5) (layer B.Cu) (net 82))
 (segment (start 120.5 119.5) (end 122 121) (width 0.5) (layer B.Cu) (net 82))
 (segment (start 131.58 116) (end 129.5 116) (width 0.5) (layer B.Cu) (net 82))
 (segment (start 129.08 116.42) (end 129.08 118.88) (width 0.5) (layer B.Cu) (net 82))
 (segment (start 129.5 116) (end 129.08 116.42) (width 0.5) (layer B.Cu) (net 82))
 (segment (start 132 116) (end 131.58 116) (width 0.5) (layer B.Cu) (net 82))
 (segment (start 134.5 118.5) (end 132 116) (width 0.5) (layer B.Cu) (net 82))
 (segment (start 135.5 118.5) (end 134.5 118.5) (width 0.5) (layer B.Cu) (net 82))
 (segment (start 136 122.5) (end 136 119) (width 0.5) (layer B.Cu) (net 82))
 (segment (start 134.5 124) (end 136 122.5) (width 0.5) (layer B.Cu) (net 82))
 (segment (start 127.5 124) (end 134.5 124) (width 0.5) (layer B.Cu) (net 82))
 (segment (start 136 119) (end 135.5 118.5) (width 0.5) (layer B.Cu) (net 82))
 (segment (start 126.54 124.96) (end 127.5 124) (width 0.5) (layer B.Cu) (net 82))
 (segment (start 126.54 126.5) (end 126.54 124.96) (width 0.5) (layer B.Cu) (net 82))
 (segment (start 119 119.5) (end 120.5 119.5) (width 0.5) (layer B.Cu) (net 82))
 (segment (start 132 131.5) (end 135.42 131.5) (width 0.5) (layer B.Cu) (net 1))
 (segment (start 128.5 134.5) (end 131 137) (width 0.5) (layer B.Cu) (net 50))
 (segment (start 127.08 134.5) (end 128.5 134.5) (width 0.5) (layer B.Cu) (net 50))
 (segment (start 128 140) (end 131 137) (width 0.5) (layer B.Cu) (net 50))
 (segment (start 128 140.5) (end 128 140) (width 0.5) (layer B.Cu) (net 50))
 (segment (start 142.5 115) (end 142.5 121.08) (width 0.5) (layer B.Cu) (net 2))
 (segment (start 141.5 114) (end 142.5 115) (width 0.5) (layer B.Cu) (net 2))
 (segment (start 140 122.04) (end 141.54 122.04) (width 0.5) (layer B.Cu) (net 2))
 (segment (start 142.96 120.62) (end 142.04 121.54) (width 0.5) (layer B.Cu) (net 2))
 (segment (start 142.04 121.54) (end 141.54 122.04) (width 0.5) (layer B.Cu) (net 2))
 (segment (start 142.5 121.08) (end 142.04 121.54) (width 0.5) (layer B.Cu) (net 2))
 (segment (start 140 131.5) (end 140 128.5) (width 0.5) (layer B.Cu) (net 2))
 (segment (start 142.5 126) (end 142.5 123) (width 0.5) (layer B.Cu) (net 2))
 (segment (start 140 128.5) (end 142.5 126) (width 0.5) (layer B.Cu) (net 2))
 (segment (start 142.5 123) (end 141.54 122.04) (width 0.5) (layer B.Cu) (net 2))
 (segment (start 138.62 137) (end 140.5 135.12) (width 0.5) (layer B.Cu) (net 2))
 (segment (start 140.5 132) (end 140 131.5) (width 0.5) (layer B.Cu) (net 2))
 (segment (start 140.5 135.12) (end 140.5 132) (width 0.5) (layer B.Cu) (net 2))
 (segment (start 119 122.5) (end 130 122.5) (width 0.5) (layer B.Cu) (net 83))
 (segment (start 131.62 120.88) (end 131.62 118.88) (width 0.5) (layer B.Cu) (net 83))
 (segment (start 131.92 120.58) (end 131.25 121.25) (width 0.5) (layer B.Cu) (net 83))
 (segment (start 134.5 120.58) (end 131.92 120.58) (width 0.5) (layer B.Cu) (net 83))
 (segment (start 131.25 121.25) (end 131.62 120.88) (width 0.5) (layer B.Cu) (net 83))
 (segment (start 130 122.5) (end 131.25 121.25) (width 0.5) (layer B.Cu) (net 83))
 (segment (start 118.5 130.96) (end 116.54 129) (width 0.5) (layer B.Cu) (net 85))
 (segment (start 116.54 129) (end 116.54 124.96) (width 0.5) (layer B.Cu) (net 85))
 (segment (start 117.73 123.77) (end 119 123.77) (width 0.5) (layer B.Cu) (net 85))
 (segment (start 116.54 124.96) (end 117.73 123.77) (width 0.5) (layer B.Cu) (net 85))
 (segment (start 138.5 119.5) (end 140 119.5) (width 0.5) (layer B.Cu) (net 79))
 (segment (start 138 124) (end 138 120) (width 0.5) (layer B.Cu) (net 79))
 (segment (start 133.5 128.5) (end 138 124) (width 0.5) (layer B.Cu) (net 79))
 (segment (start 130 128.5) (end 133.5 128.5) (width 0.5) (layer B.Cu) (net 79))
 (segment (start 129.08 127.58) (end 130 128.5) (width 0.5) (layer B.Cu) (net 79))
 (segment (start 138 120) (end 138.5 119.5) (width 0.5) (layer B.Cu) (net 79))
 (segment (start 129.08 126.5) (end 129.08 127.58) (width 0.5) (layer B.Cu) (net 79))
 (segment (start 126.5 118.84) (end 126.54 118.88) (width 0.5) (layer B.Cu) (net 81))
 (segment (start 126.5 116) (end 126.5 118.84) (width 0.5) (layer B.Cu) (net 81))
 (segment (start 126.5 115.58) (end 128.58 113.5) (width 0.5) (layer B.Cu) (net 81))
 (segment (start 126.5 116) (end 126.5 115.58) (width 0.5) (layer B.Cu) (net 81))
 (segment (start 122 133.5) (end 122 129.5) (width 0.5) (layer B.Cu) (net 84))
 (segment (start 120.92 128.42) (end 118.5 128.42) (width 0.5) (layer B.Cu) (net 84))
 (segment (start 122 129.5) (end 120.92 128.42) (width 0.5) (layer B.Cu) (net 84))
 (segment (start 122 133.5) (end 122 134.5) (width 0.5) (layer B.Cu) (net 84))
 (segment (start 113 127.42) (end 113.92 127.42) (width 0.5) (layer B.Cu) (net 86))
 (segment (start 113.92 127.42) (end 115 128.5) (width 0.5) (layer B.Cu) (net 86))
 (segment (start 115 128.5) (end 115 131) (width 0.5) (layer B.Cu) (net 86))
 (segment (start 117.5 133.5) (end 118.5 133.5) (width 0.5) (layer B.Cu) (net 86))
 (segment (start 115 131) (end 117.5 133.5) (width 0.5) (layer B.Cu) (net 86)))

